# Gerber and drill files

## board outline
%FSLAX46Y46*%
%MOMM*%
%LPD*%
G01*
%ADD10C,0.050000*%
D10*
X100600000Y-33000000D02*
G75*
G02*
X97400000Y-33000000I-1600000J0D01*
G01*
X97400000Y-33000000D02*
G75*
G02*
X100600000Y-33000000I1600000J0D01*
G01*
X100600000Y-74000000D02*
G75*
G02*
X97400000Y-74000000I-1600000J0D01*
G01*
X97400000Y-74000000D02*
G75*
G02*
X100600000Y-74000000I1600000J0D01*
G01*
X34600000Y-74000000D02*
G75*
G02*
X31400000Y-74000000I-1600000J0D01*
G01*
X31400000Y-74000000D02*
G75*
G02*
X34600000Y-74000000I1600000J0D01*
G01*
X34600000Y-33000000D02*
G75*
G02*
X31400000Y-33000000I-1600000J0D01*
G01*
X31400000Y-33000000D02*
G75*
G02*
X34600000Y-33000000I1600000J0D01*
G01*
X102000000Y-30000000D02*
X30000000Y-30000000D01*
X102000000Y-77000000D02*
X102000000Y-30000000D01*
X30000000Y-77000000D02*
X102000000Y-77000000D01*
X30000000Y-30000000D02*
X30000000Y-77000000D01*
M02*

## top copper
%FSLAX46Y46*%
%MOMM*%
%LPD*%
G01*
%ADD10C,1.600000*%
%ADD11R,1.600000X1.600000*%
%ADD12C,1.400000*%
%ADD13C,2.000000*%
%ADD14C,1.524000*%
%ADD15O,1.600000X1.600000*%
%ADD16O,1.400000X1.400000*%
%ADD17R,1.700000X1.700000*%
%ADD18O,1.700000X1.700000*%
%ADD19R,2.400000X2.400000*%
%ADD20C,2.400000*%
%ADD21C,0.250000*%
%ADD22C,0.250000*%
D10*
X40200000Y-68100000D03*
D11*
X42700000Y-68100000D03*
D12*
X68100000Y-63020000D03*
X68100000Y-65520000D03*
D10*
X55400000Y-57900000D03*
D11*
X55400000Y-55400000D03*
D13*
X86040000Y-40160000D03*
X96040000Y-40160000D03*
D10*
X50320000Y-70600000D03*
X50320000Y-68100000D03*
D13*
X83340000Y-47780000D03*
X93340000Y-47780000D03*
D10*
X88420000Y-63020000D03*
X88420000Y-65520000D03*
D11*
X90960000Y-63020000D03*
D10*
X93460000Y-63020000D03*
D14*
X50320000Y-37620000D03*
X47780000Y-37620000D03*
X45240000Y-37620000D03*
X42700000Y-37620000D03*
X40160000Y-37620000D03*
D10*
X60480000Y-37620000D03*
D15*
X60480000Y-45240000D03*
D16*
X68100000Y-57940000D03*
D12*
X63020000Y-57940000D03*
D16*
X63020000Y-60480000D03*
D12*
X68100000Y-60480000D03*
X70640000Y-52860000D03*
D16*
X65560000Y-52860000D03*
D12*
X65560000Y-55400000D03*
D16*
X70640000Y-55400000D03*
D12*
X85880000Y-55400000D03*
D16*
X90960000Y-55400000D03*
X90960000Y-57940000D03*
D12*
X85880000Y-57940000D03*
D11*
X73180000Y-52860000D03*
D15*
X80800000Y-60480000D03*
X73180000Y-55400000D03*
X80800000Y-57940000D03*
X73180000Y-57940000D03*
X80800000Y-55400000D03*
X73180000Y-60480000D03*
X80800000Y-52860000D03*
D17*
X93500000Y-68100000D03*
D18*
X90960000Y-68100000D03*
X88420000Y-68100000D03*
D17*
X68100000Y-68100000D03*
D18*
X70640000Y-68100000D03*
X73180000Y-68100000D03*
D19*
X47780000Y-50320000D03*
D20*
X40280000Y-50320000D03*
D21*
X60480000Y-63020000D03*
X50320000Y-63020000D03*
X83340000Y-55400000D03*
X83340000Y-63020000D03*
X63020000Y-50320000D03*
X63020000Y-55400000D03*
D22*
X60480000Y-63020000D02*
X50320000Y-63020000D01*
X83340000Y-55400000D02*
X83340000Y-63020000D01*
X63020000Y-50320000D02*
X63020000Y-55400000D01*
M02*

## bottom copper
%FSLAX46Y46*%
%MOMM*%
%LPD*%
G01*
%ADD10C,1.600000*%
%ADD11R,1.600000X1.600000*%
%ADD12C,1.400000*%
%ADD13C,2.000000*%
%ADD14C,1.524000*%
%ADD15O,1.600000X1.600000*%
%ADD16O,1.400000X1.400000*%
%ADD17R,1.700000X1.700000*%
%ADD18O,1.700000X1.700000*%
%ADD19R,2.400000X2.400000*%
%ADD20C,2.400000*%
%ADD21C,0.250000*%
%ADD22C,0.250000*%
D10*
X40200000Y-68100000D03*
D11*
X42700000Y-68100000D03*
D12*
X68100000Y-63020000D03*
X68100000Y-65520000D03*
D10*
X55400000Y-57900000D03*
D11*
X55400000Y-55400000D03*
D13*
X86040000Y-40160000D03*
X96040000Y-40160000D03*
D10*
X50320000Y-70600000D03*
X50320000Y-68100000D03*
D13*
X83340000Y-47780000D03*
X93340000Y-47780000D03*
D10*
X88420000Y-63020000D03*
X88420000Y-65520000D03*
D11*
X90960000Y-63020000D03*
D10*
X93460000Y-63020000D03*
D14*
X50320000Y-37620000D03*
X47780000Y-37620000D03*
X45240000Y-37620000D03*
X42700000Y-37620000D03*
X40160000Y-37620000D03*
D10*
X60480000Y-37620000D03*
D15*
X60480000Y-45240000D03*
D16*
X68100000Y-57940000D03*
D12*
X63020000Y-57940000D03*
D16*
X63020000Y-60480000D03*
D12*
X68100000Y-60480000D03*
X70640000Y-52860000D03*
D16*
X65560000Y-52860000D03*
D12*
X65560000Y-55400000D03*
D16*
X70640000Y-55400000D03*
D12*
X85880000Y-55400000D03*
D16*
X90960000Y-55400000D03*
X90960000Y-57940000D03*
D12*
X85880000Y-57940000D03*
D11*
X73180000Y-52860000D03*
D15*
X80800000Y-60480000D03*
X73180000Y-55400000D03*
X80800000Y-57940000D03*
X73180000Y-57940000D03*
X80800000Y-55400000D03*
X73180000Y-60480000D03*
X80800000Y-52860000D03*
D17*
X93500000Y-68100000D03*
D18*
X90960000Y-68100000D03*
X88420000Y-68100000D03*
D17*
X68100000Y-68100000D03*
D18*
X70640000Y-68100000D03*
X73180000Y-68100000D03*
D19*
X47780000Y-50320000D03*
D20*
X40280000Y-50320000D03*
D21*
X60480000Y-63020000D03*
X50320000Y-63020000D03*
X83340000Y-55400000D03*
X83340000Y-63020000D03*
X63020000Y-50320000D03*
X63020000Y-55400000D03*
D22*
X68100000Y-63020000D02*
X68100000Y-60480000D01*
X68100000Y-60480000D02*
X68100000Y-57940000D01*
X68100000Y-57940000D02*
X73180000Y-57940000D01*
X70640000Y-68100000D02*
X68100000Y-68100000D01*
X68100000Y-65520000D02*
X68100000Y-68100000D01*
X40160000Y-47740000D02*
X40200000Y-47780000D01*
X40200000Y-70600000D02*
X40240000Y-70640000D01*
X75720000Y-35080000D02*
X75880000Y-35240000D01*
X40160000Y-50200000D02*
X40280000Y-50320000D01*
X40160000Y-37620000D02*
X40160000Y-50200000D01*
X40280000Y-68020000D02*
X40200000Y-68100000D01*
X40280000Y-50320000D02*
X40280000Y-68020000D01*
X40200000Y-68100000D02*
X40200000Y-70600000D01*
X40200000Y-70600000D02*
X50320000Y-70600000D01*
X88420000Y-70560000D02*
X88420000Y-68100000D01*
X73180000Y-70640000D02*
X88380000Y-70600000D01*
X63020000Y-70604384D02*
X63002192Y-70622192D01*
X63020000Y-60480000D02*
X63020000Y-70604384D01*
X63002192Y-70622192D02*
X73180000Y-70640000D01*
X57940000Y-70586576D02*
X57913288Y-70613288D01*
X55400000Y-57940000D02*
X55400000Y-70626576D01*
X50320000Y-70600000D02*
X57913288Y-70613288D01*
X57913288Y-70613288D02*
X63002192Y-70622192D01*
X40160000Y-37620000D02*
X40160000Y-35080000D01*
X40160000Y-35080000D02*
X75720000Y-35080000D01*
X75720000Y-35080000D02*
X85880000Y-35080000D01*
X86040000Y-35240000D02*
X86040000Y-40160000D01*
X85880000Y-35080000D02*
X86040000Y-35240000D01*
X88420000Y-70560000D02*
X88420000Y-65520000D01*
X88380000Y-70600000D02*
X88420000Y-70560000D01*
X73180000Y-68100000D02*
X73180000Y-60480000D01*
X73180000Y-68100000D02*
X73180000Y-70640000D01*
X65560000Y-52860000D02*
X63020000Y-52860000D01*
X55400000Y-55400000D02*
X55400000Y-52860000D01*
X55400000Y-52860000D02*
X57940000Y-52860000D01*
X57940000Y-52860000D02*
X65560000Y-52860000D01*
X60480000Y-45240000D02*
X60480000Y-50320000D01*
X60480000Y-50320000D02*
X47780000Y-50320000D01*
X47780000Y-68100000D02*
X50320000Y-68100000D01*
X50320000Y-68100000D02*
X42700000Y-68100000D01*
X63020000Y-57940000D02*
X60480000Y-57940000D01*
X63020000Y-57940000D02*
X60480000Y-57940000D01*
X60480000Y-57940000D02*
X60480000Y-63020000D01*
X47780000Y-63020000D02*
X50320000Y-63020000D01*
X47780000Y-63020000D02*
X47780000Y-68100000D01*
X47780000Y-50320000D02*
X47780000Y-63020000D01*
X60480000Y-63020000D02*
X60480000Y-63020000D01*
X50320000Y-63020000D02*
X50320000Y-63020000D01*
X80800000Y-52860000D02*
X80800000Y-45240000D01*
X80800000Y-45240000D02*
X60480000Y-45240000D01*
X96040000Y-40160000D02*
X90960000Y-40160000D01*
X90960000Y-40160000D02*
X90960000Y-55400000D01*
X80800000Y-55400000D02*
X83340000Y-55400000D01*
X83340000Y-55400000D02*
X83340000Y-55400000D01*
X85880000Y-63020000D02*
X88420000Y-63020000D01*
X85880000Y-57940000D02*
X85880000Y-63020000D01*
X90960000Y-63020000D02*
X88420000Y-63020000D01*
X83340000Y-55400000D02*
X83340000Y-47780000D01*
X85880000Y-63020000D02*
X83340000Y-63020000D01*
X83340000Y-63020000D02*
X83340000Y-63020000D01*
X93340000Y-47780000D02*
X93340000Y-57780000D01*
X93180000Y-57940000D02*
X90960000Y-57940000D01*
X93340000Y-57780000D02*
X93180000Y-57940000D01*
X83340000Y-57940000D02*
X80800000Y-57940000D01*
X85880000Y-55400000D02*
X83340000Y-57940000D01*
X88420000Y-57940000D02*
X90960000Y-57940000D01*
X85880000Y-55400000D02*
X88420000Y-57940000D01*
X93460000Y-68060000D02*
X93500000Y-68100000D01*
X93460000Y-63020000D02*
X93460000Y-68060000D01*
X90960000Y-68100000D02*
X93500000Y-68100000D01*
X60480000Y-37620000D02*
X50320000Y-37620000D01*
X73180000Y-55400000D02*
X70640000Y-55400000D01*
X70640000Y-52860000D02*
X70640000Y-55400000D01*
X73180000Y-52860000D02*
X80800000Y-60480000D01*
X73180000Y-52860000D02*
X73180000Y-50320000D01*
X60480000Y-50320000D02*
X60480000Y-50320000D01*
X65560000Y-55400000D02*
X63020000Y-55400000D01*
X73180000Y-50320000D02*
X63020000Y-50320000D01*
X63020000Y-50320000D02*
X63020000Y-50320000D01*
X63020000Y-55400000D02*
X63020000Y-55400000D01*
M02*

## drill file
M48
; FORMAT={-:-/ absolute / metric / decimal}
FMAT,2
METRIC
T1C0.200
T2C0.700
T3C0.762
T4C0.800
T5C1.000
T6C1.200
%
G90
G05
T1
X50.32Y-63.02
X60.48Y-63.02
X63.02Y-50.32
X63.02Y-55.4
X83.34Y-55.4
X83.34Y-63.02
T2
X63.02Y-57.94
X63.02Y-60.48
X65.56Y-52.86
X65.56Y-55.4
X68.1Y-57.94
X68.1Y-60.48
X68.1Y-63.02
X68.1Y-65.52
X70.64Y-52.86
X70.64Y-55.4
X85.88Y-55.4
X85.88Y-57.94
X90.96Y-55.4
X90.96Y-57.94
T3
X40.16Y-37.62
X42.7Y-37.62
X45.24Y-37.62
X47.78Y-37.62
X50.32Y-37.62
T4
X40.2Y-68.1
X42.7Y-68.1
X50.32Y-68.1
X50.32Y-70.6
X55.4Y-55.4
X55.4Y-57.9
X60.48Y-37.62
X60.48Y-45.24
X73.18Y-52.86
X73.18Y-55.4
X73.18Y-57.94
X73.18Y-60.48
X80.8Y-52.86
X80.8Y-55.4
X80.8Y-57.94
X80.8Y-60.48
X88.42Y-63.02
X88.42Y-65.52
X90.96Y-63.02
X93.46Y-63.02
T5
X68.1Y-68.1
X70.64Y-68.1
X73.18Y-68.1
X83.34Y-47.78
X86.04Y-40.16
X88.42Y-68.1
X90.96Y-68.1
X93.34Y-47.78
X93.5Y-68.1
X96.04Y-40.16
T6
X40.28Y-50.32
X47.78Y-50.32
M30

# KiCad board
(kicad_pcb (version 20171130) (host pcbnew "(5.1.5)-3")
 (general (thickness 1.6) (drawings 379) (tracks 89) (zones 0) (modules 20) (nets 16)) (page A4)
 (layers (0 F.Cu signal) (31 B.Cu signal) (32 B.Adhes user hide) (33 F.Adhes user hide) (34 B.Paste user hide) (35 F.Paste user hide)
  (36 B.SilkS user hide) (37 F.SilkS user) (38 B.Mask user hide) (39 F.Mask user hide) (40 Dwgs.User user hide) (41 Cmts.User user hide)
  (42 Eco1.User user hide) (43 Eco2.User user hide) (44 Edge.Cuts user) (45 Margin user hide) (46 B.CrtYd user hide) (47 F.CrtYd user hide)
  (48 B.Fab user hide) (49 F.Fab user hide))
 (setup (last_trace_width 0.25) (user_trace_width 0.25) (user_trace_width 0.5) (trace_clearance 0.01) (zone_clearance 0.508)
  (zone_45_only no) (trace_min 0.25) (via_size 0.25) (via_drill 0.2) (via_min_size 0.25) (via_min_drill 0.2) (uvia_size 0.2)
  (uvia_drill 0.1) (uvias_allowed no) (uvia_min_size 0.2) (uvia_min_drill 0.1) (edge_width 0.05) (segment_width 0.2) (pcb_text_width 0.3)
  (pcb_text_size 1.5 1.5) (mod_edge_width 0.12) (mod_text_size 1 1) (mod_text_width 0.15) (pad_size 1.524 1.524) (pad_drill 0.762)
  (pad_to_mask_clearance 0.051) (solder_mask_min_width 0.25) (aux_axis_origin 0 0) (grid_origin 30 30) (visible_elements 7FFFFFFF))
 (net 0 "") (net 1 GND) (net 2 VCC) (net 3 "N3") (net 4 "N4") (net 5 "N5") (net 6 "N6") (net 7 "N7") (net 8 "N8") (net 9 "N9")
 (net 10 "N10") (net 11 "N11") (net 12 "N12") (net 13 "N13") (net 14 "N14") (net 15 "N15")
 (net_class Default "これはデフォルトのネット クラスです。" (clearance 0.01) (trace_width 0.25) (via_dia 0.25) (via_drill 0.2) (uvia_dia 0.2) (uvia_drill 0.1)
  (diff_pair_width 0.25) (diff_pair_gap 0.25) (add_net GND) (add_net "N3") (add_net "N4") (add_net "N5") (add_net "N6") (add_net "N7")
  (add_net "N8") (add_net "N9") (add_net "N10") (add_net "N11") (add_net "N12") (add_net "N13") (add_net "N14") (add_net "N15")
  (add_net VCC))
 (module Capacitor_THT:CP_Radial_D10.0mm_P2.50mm (layer F.Cu) (at 42.7 68.1 180)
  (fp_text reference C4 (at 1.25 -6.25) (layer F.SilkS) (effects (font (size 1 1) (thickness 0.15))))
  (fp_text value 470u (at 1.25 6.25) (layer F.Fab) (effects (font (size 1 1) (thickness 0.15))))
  (pad 2 thru_hole circle (at 2.5 0 180) (size 1.6 1.6) (drill 0.8) (layers *.Cu *.Mask) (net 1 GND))
  (pad 1 thru_hole rect (at 0 0 180) (size 1.6 1.6) (drill 0.8) (layers *.Cu *.Mask) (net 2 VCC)))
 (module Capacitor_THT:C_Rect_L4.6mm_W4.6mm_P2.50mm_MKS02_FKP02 (layer F.Cu) (at 68.1 63.02 270)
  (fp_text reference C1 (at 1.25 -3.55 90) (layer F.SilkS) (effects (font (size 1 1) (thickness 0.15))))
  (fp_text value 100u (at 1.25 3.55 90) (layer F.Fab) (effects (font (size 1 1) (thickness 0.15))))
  (pad 1 thru_hole circle (at 0 0 270) (size 1.4 1.4) (drill 0.7) (layers *.Cu *.Mask) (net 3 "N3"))
  (pad 2 thru_hole circle (at 2.5 0 270) (size 1.4 1.4) (drill 0.7) (layers *.Cu *.Mask) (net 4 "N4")))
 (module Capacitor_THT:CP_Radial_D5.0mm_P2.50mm (layer F.Cu) (at 55.4 55.4 270)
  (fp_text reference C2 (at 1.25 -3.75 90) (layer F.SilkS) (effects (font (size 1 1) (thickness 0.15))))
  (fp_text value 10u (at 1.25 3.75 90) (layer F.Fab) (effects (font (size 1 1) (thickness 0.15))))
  (pad 2 thru_hole circle (at 2.5 0 270) (size 1.6 1.6) (drill 0.8) (layers *.Cu *.Mask) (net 1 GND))
  (pad 1 thru_hole rect (at 0 0 270) (size 1.6 1.6) (drill 0.8) (layers *.Cu *.Mask) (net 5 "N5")))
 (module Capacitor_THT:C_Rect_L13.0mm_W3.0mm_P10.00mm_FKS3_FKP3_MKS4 (layer F.Cu) (at 96.04 40.16 180)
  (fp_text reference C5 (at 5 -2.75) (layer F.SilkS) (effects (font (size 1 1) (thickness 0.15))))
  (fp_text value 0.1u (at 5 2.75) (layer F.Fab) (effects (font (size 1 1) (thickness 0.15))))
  (pad 2 thru_hole circle (at 10 0 180) (size 2 2) (drill 1) (layers *.Cu *.Mask) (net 1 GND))
  (pad 1 thru_hole circle (at 0 0 180) (size 2 2) (drill 1) (layers *.Cu *.Mask) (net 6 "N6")))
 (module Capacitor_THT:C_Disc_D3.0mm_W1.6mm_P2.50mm (layer F.Cu) (at 50.32 68.1 270)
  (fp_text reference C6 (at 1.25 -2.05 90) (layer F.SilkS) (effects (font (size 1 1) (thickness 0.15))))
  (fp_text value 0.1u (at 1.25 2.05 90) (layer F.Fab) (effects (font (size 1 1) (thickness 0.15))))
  (pad 2 thru_hole circle (at 2.5 0 270) (size 1.6 1.6) (drill 0.8) (layers *.Cu *.Mask) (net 1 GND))
  (pad 1 thru_hole circle (at 0 0 270) (size 1.6 1.6) (drill 0.8) (layers *.Cu *.Mask) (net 2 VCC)))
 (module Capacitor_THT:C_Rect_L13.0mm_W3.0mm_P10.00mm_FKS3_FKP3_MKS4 (layer F.Cu) (at 83.34 47.78)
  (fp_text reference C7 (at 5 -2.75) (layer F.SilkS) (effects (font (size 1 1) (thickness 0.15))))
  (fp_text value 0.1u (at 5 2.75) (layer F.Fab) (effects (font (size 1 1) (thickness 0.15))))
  (pad 1 thru_hole circle (at 0 0) (size 2 2) (drill 1) (layers *.Cu *.Mask) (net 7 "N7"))
  (pad 2 thru_hole circle (at 10 0) (size 2 2) (drill 1) (layers *.Cu *.Mask) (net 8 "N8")))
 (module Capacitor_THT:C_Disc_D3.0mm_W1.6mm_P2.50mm (layer F.Cu) (at 88.42 63.02 270)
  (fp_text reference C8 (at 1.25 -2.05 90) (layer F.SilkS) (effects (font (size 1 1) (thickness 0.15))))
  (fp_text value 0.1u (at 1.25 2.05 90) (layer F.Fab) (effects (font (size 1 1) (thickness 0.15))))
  (pad 1 thru_hole circle (at 0 0 270) (size 1.6 1.6) (drill 0.8) (layers *.Cu *.Mask) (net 7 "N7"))
  (pad 2 thru_hole circle (at 2.5 0 270) (size 1.6 1.6) (drill 0.8) (layers *.Cu *.Mask) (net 1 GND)))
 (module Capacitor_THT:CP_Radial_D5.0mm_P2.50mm (layer F.Cu) (at 90.96 63.02)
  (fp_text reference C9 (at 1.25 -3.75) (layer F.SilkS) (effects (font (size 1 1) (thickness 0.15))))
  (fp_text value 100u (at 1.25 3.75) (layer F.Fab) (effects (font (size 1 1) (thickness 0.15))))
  (pad 1 thru_hole rect (at 0 0) (size 1.6 1.6) (drill 0.8) (layers *.Cu *.Mask) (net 7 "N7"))
  (pad 2 thru_hole circle (at 2.5 0) (size 1.6 1.6) (drill 0.8) (layers *.Cu *.Mask) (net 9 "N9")))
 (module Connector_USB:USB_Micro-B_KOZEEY (layer F.Cu) (at 40.16 37.62)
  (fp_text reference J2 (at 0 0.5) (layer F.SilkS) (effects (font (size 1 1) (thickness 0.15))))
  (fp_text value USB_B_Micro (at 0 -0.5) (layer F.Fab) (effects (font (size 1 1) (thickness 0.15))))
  (pad 1 thru_hole circle (at 10.16 0) (size 1.524 1.524) (drill 0.762) (layers *.Cu *.Mask) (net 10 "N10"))
  (pad 2 thru_hole circle (at 7.62 0) (size 1.524 1.524) (drill 0.762) (layers *.Cu *.Mask) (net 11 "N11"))
  (pad 3 thru_hole circle (at 5.08 0) (size 1.524 1.524) (drill 0.762) (layers *.Cu *.Mask) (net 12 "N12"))
  (pad 4 thru_hole circle (at 2.54 0) (size 1.524 1.524) (drill 0.762) (layers *.Cu *.Mask) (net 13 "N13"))
  (pad 5 thru_hole circle (at 0 0) (size 1.524 1.524) (drill 0.762) (layers *.Cu *.Mask) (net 1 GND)))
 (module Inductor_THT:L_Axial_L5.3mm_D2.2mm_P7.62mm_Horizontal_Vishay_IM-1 (layer F.Cu) (at 60.48 37.62 270)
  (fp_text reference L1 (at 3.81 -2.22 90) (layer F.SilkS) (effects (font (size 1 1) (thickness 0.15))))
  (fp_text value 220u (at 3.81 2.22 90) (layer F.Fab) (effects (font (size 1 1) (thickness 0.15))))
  (pad 1 thru_hole circle (at 0 0 270) (size 1.6 1.6) (drill 0.8) (layers *.Cu *.Mask) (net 10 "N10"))
  (pad 2 thru_hole oval (at 7.62 0 270) (size 1.6 1.6) (drill 0.8) (layers *.Cu *.Mask) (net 2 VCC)))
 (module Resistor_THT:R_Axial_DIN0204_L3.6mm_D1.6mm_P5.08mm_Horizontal (layer F.Cu) (at 63.02 57.94)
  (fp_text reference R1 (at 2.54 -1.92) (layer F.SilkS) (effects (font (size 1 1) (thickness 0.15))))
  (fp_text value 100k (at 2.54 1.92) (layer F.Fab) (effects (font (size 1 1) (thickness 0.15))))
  (pad 2 thru_hole oval (at 5.08 0) (size 1.4 1.4) (drill 0.7) (layers *.Cu *.Mask) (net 3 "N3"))
  (pad 1 thru_hole circle (at 0 0) (size 1.4 1.4) (drill 0.7) (layers *.Cu *.Mask) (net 2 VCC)))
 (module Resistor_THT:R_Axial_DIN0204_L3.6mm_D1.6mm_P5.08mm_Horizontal (layer F.Cu) (at 68.1 60.48 180)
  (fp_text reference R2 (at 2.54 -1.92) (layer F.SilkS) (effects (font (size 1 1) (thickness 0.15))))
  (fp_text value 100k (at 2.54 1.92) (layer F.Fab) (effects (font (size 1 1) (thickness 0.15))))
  (pad 2 thru_hole oval (at 5.08 0 180) (size 1.4 1.4) (drill 0.7) (layers *.Cu *.Mask) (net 1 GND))
  (pad 1 thru_hole circle (at 0 0 180) (size 1.4 1.4) (drill 0.7) (layers *.Cu *.Mask) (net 3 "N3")))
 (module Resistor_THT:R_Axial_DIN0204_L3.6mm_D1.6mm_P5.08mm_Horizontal (layer F.Cu) (at 70.64 52.86 180)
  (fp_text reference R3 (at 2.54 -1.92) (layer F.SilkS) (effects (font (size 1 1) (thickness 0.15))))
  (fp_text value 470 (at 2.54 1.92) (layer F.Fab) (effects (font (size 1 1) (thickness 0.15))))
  (pad 1 thru_hole circle (at 0 0 180) (size 1.4 1.4) (drill 0.7) (layers *.Cu *.Mask) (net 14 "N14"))
  (pad 2 thru_hole oval (at 5.08 0 180) (size 1.4 1.4) (drill 0.7) (layers *.Cu *.Mask) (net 5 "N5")))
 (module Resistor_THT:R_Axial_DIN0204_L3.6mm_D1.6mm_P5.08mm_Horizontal (layer F.Cu) (at 65.56 55.4)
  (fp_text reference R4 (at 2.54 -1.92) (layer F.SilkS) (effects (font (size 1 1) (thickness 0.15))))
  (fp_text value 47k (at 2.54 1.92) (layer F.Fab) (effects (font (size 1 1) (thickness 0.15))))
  (pad 1 thru_hole circle (at 0 0) (size 1.4 1.4) (drill 0.7) (layers *.Cu *.Mask) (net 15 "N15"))
  (pad 2 thru_hole oval (at 5.08 0) (size 1.4 1.4) (drill 0.7) (layers *.Cu *.Mask) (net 14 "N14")))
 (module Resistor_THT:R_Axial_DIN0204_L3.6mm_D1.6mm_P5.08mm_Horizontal (layer F.Cu) (at 85.88 55.4)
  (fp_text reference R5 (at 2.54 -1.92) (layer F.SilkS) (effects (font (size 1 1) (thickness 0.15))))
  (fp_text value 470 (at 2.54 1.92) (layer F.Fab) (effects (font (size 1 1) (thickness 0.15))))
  (pad 1 thru_hole circle (at 0 0) (size 1.4 1.4) (drill 0.7) (layers *.Cu *.Mask) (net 8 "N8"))
  (pad 2 thru_hole oval (at 5.08 0) (size 1.4 1.4) (drill 0.7) (layers *.Cu *.Mask) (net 6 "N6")))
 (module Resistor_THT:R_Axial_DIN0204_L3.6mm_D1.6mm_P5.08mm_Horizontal (layer F.Cu) (at 85.88 57.94)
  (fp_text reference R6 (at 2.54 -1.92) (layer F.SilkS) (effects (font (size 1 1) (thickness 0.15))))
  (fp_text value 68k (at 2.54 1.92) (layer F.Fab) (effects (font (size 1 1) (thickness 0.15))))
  (pad 2 thru_hole oval (at 5.08 0) (size 1.4 1.4) (drill 0.7) (layers *.Cu *.Mask) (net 8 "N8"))
  (pad 1 thru_hole circle (at 0 0) (size 1.4 1.4) (drill 0.7) (layers *.Cu *.Mask) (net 7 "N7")))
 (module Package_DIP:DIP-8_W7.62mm (layer F.Cu) (at 73.18 52.86)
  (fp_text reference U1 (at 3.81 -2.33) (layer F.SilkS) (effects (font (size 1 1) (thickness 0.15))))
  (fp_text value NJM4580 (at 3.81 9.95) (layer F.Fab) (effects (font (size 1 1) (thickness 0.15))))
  (pad 1 thru_hole rect (at 0 0) (size 1.6 1.6) (drill 0.8) (layers *.Cu *.Mask) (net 15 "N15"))
  (pad 5 thru_hole oval (at 7.62 7.62) (size 1.6 1.6) (drill 0.8) (layers *.Cu *.Mask) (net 15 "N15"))
  (pad 2 thru_hole oval (at 0 2.54) (size 1.6 1.6) (drill 0.8) (layers *.Cu *.Mask) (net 14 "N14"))
  (pad 6 thru_hole oval (at 7.62 5.08) (size 1.6 1.6) (drill 0.8) (layers *.Cu *.Mask) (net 8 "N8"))
  (pad 3 thru_hole oval (at 0 5.08) (size 1.6 1.6) (drill 0.8) (layers *.Cu *.Mask) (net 3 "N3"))
  (pad 7 thru_hole oval (at 7.62 2.54) (size 1.6 1.6) (drill 0.8) (layers *.Cu *.Mask) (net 7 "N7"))
  (pad 4 thru_hole oval (at 0 7.62) (size 1.6 1.6) (drill 0.8) (layers *.Cu *.Mask) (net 1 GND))
  (pad 8 thru_hole oval (at 7.62 0) (size 1.6 1.6) (drill 0.8) (layers *.Cu *.Mask) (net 2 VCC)))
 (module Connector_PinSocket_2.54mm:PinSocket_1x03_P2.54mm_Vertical (layer F.Cu) (at 93.5 68.1 270)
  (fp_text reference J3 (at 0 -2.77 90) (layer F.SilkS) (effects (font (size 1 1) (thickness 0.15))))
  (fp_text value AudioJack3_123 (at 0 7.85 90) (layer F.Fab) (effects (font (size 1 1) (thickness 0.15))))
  (pad 1 thru_hole rect (at 0 0 270) (size 1.7 1.7) (drill 1) (layers *.Cu *.Mask) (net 9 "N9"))
  (pad 2 thru_hole oval (at 0 2.54 270) (size 1.7 1.7) (drill 1) (layers *.Cu *.Mask) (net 9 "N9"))
  (pad 3 thru_hole oval (at 0 5.08 270) (size 1.7 1.7) (drill 1) (layers *.Cu *.Mask) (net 1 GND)))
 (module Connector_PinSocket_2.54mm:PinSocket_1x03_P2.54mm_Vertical (layer F.Cu) (at 68.1 68.1 90)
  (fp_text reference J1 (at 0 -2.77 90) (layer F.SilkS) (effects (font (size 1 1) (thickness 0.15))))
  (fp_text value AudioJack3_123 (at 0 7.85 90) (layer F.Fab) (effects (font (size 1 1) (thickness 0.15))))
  (pad 1 thru_hole rect (at 0 0 90) (size 1.7 1.7) (drill 1) (layers *.Cu *.Mask) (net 4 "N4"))
  (pad 2 thru_hole oval (at 0 2.54 90) (size 1.7 1.7) (drill 1) (layers *.Cu *.Mask) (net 4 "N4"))
  (pad 3 thru_hole oval (at 0 5.08 90) (size 1.7 1.7) (drill 1) (layers *.Cu *.Mask) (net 1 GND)))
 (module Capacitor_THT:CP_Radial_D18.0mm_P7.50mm (layer F.Cu) (at 47.78 50.32 180)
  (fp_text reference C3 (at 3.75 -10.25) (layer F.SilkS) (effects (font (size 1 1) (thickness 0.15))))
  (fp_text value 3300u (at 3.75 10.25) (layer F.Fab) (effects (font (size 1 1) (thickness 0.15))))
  (pad 1 thru_hole rect (at 0 0 180) (size 2.4 2.4) (drill 1.2) (layers *.Cu *.Mask) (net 2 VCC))
  (pad 2 thru_hole circle (at 7.5 0 180) (size 2.4 2.4) (drill 1.2) (layers *.Cu *.Mask) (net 1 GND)))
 (gr_circle (center 99 33) (end 99 34.6) (layer Edge.Cuts) (width 0.05))
 (gr_circle (center 99 74) (end 99 75.6) (layer Edge.Cuts) (width 0.05))
 (gr_circle (center 33 74) (end 33 75.6) (layer Edge.Cuts) (width 0.05))
 (gr_circle (center 33 33) (end 33 34.6) (layer Edge.Cuts) (width 0.05))
 (gr_line (start 102 30) (end 30 30) (layer Edge.Cuts) (width 0.05))
 (gr_line (start 102 77) (end 102 30) (layer Edge.Cuts) (width 0.05))
 (gr_line (start 30 77) (end 102 77) (layer Edge.Cuts) (width 0.05))
 (gr_line (start 30 30) (end 30 77) (layer Edge.Cuts) (width 0.05))
 (segment (start 68.1 63.02) (end 68.1 60.48) (width 0.25) (layer B.Cu) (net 3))
 (segment (start 68.1 60.48) (end 68.1 57.94) (width 0.25) (layer B.Cu) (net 3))
 (segment (start 68.1 57.94) (end 73.18 57.94) (width 0.25) (layer B.Cu) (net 3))
 (segment (start 70.64 68.1) (end 68.1 68.1) (width 0.25) (layer B.Cu) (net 4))
 (segment (start 68.1 65.52) (end 68.1 68.1) (width 0.25) (layer B.Cu) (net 4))
 (segment (start 40.16 47.74) (end 40.2 47.78) (width 0.25) (layer B.Cu) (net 1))
 (segment (start 40.2 70.6) (end 40.24 70.64) (width 0.25) (layer B.Cu) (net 1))
 (segment (start 75.72 35.08) (end 75.88 35.24) (width 0.25) (layer B.Cu) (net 1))
 (segment (start 40.16 50.2) (end 40.28 50.32) (width 0.25) (layer B.Cu) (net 1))
 (segment (start 40.16 37.62) (end 40.16 50.2) (width 0.25) (layer B.Cu) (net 1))
 (segment (start 40.28 68.02) (end 40.2 68.1) (width 0.25) (layer B.Cu) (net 1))
 (segment (start 40.28 50.32) (end 40.28 68.02) (width 0.25) (layer B.Cu) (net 1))
 (segment (start 40.2 68.1) (end 40.2 70.6) (width 0.25) (layer B.Cu) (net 1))
 (segment (start 40.2 70.6) (end 50.32 70.6) (width 0.25) (layer B.Cu) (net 1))
 (segment (start 88.42 70.56) (end 88.42 68.1) (width 0.25) (layer B.Cu) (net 1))
 (segment (start 73.18 70.64) (end 88.38 70.6) (width 0.25) (layer B.Cu) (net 1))
 (segment (start 63.02 70.604384) (end 63.002192 70.622192) (width 0.25) (layer B.Cu) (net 1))
 (segment (start 63.02 60.48) (end 63.02 70.604384) (width 0.25) (layer B.Cu) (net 1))
 (segment (start 63.002192 70.622192) (end 73.18 70.64) (width 0.25) (layer B.Cu) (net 1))
 (segment (start 57.94 70.586576) (end 57.913288 70.613288) (width 0.25) (layer B.Cu) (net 1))
 (segment (start 55.4 57.94) (end 55.4 70.626576) (width 0.25) (layer B.Cu) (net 1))
 (segment (start 50.32 70.6) (end 57.913288 70.613288) (width 0.25) (layer B.Cu) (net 1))
 (segment (start 57.913288 70.613288) (end 63.002192 70.622192) (width 0.25) (layer B.Cu) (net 1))
 (segment (start 40.16 37.62) (end 40.16 35.08) (width 0.25) (layer B.Cu) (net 1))
 (segment (start 40.16 35.08) (end 75.72 35.08) (width 0.25) (layer B.Cu) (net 1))
 (segment (start 75.72 35.08) (end 85.88 35.08) (width 0.25) (layer B.Cu) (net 1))
 (segment (start 86.04 35.24) (end 86.04 40.16) (width 0.25) (layer B.Cu) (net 1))
 (segment (start 85.88 35.08) (end 86.04 35.24) (width 0.25) (layer B.Cu) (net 1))
 (segment (start 88.42 70.56) (end 88.42 65.52) (width 0.25) (layer B.Cu) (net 1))
 (segment (start 88.38 70.6) (end 88.42 70.56) (width 0.25) (layer B.Cu) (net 1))
 (segment (start 73.18 68.1) (end 73.18 60.48) (width 0.25) (layer B.Cu) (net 1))
 (segment (start 73.18 68.1) (end 73.18 70.64) (width 0.25) (layer B.Cu) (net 1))
 (segment (start 65.56 52.86) (end 63.02 52.86) (width 0.25) (layer B.Cu) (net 5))
 (segment (start 55.4 55.4) (end 55.4 52.86) (width 0.25) (layer B.Cu) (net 5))
 (segment (start 55.4 52.86) (end 57.94 52.86) (width 0.25) (layer B.Cu) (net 5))
 (segment (start 57.94 52.86) (end 65.56 52.86) (width 0.25) (layer B.Cu) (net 5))
 (segment (start 60.48 45.24) (end 60.48 50.32) (width 0.25) (layer B.Cu) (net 2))
 (segment (start 60.48 50.32) (end 47.78 50.32) (width 0.25) (layer B.Cu) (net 2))
 (segment (start 47.78 68.1) (end 50.32 68.1) (width 0.25) (layer B.Cu) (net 2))
 (segment (start 50.32 68.1) (end 42.7 68.1) (width 0.25) (layer B.Cu) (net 2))
 (segment (start 63.02 57.94) (end 60.48 57.94) (width 0.25) (layer B.Cu) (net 2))
 (segment (start 63.02 57.94) (end 60.48 57.94) (width 0.25) (layer B.Cu) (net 2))
 (segment (start 60.48 57.94) (end 60.48 63.02) (width 0.25) (layer B.Cu) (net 2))
 (segment (start 47.78 63.02) (end 50.32 63.02) (width 0.25) (layer B.Cu) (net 2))
 (segment (start 47.78 63.02) (end 47.78 68.1) (width 0.25) (layer B.Cu) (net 2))
 (segment (start 47.78 50.32) (end 47.78 63.02) (width 0.25) (layer B.Cu) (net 2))
 (segment (start 60.48 63.02) (end 60.48 63.02) (width 0.25) (layer B.Cu) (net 2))
 (via (at 60.48 63.02) (size 0.25) (drill 0.2) (layers F.Cu B.Cu) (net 2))
 (segment (start 50.32 63.02) (end 50.32 63.02) (width 0.25) (layer B.Cu) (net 2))
 (via (at 50.32 63.02) (size 0.25) (drill 0.2) (layers F.Cu B.Cu) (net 2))
 (segment (start 60.48 63.02) (end 50.32 63.02) (width 0.25) (layer F.Cu) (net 2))
 (segment (start 80.8 52.86) (end 80.8 45.24) (width 0.25) (layer B.Cu) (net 2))
 (segment (start 80.8 45.24) (end 60.48 45.24) (width 0.25) (layer B.Cu) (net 2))
 (segment (start 96.04 40.16) (end 90.96 40.16) (width 0.25) (layer B.Cu) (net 6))
 (segment (start 90.96 40.16) (end 90.96 55.4) (width 0.25) (layer B.Cu) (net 6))
 (segment (start 80.8 55.4) (end 83.34 55.4) (width 0.25) (layer B.Cu) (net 7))
 (segment (start 83.34 55.4) (end 83.34 55.4) (width 0.25) (layer B.Cu) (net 7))
 (segment (start 85.88 63.02) (end 88.42 63.02) (width 0.25) (layer B.Cu) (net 7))
 (segment (start 85.88 57.94) (end 85.88 63.02) (width 0.25) (layer B.Cu) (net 7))
 (segment (start 90.96 63.02) (end 88.42 63.02) (width 0.25) (layer B.Cu) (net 7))
 (segment (start 83.34 55.4) (end 83.34 47.78) (width 0.25) (layer B.Cu) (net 7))
 (via (at 83.34 55.4) (size 0.25) (drill 0.2) (layers F.Cu B.Cu) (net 7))
 (segment (start 85.88 63.02) (end 83.34 63.02) (width 0.25) (layer B.Cu) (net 7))
 (segment (start 83.34 63.02) (end 83.34 63.02) (width 0.25) (layer B.Cu) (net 7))
 (via (at 83.34 63.02) (size 0.25) (drill 0.2) (layers F.Cu B.Cu) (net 7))
 (segment (start 83.34 55.4) (end 83.34 63.02) (width 0.25) (layer F.Cu) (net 7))
 (segment (start 93.34 47.78) (end 93.34 57.78) (width 0.25) (layer B.Cu) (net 8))
 (segment (start 93.18 57.94) (end 90.96 57.94) (width 0.25) (layer B.Cu) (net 8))
 (segment (start 93.34 57.78) (end 93.18 57.94) (width 0.25) (layer B.Cu) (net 8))
 (segment (start 83.34 57.94) (end 80.8 57.94) (width 0.25) (layer B.Cu) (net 8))
 (segment (start 85.88 55.4) (end 83.34 57.94) (width 0.25) (layer B.Cu) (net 8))
 (segment (start 88.42 57.94) (end 90.96 57.94) (width 0.25) (layer B.Cu) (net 8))
 (segment (start 85.88 55.4) (end 88.42 57.94) (width 0.25) (layer B.Cu) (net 8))
 (segment (start 93.46 68.06) (end 93.5 68.1) (width 0.25) (layer B.Cu) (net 9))
 (segment (start 93.46 63.02) (end 93.46 68.06) (width 0.25) (layer B.Cu) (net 9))
 (segment (start 90.96 68.1) (end 93.5 68.1) (width 0.25) (layer B.Cu) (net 9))
 (segment (start 60.48 37.62) (end 50.32 37.62) (width 0.25) (layer B.Cu) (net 10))
 (segment (start 73.18 55.4) (end 70.64 55.4) (width 0.25) (layer B.Cu) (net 14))
 (segment (start 70.64 52.86) (end 70.64 55.4) (width 0.25) (layer B.Cu) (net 14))
 (segment (start 73.18 52.86) (end 80.8 60.48) (width 0.25) (layer B.Cu) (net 15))
 (segment (start 73.18 52.86) (end 73.18 50.32) (width 0.25) (layer B.Cu) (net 15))
 (segment (start 60.48 50.32) (end 60.48 50.32) (width 0.25) (layer B.Cu) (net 2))
 (segment (start 63.02 50.32) (end 63.02 55.4) (width 0.25) (layer F.Cu) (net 15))
 (segment (start 65.56 55.4) (end 63.02 55.4) (width 0.25) (layer B.Cu) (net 15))
 (segment (start 73.18 50.32) (end 63.02 50.32) (width 0.25) (layer B.Cu) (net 15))
 (segment (start 63.02 50.32) (end 63.02 50.32) (width 0.25) (layer B.Cu) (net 15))
 (via (at 63.02 50.32) (size 0.25) (drill 0.2) (layers F.Cu B.Cu) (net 15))
 (segment (start 63.02 55.4) (end 63.02 55.4) (width 0.25) (layer B.Cu) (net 15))
 (via (at 63.02 55.4) (size 0.25) (drill 0.2) (layers F.Cu B.Cu) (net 15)))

